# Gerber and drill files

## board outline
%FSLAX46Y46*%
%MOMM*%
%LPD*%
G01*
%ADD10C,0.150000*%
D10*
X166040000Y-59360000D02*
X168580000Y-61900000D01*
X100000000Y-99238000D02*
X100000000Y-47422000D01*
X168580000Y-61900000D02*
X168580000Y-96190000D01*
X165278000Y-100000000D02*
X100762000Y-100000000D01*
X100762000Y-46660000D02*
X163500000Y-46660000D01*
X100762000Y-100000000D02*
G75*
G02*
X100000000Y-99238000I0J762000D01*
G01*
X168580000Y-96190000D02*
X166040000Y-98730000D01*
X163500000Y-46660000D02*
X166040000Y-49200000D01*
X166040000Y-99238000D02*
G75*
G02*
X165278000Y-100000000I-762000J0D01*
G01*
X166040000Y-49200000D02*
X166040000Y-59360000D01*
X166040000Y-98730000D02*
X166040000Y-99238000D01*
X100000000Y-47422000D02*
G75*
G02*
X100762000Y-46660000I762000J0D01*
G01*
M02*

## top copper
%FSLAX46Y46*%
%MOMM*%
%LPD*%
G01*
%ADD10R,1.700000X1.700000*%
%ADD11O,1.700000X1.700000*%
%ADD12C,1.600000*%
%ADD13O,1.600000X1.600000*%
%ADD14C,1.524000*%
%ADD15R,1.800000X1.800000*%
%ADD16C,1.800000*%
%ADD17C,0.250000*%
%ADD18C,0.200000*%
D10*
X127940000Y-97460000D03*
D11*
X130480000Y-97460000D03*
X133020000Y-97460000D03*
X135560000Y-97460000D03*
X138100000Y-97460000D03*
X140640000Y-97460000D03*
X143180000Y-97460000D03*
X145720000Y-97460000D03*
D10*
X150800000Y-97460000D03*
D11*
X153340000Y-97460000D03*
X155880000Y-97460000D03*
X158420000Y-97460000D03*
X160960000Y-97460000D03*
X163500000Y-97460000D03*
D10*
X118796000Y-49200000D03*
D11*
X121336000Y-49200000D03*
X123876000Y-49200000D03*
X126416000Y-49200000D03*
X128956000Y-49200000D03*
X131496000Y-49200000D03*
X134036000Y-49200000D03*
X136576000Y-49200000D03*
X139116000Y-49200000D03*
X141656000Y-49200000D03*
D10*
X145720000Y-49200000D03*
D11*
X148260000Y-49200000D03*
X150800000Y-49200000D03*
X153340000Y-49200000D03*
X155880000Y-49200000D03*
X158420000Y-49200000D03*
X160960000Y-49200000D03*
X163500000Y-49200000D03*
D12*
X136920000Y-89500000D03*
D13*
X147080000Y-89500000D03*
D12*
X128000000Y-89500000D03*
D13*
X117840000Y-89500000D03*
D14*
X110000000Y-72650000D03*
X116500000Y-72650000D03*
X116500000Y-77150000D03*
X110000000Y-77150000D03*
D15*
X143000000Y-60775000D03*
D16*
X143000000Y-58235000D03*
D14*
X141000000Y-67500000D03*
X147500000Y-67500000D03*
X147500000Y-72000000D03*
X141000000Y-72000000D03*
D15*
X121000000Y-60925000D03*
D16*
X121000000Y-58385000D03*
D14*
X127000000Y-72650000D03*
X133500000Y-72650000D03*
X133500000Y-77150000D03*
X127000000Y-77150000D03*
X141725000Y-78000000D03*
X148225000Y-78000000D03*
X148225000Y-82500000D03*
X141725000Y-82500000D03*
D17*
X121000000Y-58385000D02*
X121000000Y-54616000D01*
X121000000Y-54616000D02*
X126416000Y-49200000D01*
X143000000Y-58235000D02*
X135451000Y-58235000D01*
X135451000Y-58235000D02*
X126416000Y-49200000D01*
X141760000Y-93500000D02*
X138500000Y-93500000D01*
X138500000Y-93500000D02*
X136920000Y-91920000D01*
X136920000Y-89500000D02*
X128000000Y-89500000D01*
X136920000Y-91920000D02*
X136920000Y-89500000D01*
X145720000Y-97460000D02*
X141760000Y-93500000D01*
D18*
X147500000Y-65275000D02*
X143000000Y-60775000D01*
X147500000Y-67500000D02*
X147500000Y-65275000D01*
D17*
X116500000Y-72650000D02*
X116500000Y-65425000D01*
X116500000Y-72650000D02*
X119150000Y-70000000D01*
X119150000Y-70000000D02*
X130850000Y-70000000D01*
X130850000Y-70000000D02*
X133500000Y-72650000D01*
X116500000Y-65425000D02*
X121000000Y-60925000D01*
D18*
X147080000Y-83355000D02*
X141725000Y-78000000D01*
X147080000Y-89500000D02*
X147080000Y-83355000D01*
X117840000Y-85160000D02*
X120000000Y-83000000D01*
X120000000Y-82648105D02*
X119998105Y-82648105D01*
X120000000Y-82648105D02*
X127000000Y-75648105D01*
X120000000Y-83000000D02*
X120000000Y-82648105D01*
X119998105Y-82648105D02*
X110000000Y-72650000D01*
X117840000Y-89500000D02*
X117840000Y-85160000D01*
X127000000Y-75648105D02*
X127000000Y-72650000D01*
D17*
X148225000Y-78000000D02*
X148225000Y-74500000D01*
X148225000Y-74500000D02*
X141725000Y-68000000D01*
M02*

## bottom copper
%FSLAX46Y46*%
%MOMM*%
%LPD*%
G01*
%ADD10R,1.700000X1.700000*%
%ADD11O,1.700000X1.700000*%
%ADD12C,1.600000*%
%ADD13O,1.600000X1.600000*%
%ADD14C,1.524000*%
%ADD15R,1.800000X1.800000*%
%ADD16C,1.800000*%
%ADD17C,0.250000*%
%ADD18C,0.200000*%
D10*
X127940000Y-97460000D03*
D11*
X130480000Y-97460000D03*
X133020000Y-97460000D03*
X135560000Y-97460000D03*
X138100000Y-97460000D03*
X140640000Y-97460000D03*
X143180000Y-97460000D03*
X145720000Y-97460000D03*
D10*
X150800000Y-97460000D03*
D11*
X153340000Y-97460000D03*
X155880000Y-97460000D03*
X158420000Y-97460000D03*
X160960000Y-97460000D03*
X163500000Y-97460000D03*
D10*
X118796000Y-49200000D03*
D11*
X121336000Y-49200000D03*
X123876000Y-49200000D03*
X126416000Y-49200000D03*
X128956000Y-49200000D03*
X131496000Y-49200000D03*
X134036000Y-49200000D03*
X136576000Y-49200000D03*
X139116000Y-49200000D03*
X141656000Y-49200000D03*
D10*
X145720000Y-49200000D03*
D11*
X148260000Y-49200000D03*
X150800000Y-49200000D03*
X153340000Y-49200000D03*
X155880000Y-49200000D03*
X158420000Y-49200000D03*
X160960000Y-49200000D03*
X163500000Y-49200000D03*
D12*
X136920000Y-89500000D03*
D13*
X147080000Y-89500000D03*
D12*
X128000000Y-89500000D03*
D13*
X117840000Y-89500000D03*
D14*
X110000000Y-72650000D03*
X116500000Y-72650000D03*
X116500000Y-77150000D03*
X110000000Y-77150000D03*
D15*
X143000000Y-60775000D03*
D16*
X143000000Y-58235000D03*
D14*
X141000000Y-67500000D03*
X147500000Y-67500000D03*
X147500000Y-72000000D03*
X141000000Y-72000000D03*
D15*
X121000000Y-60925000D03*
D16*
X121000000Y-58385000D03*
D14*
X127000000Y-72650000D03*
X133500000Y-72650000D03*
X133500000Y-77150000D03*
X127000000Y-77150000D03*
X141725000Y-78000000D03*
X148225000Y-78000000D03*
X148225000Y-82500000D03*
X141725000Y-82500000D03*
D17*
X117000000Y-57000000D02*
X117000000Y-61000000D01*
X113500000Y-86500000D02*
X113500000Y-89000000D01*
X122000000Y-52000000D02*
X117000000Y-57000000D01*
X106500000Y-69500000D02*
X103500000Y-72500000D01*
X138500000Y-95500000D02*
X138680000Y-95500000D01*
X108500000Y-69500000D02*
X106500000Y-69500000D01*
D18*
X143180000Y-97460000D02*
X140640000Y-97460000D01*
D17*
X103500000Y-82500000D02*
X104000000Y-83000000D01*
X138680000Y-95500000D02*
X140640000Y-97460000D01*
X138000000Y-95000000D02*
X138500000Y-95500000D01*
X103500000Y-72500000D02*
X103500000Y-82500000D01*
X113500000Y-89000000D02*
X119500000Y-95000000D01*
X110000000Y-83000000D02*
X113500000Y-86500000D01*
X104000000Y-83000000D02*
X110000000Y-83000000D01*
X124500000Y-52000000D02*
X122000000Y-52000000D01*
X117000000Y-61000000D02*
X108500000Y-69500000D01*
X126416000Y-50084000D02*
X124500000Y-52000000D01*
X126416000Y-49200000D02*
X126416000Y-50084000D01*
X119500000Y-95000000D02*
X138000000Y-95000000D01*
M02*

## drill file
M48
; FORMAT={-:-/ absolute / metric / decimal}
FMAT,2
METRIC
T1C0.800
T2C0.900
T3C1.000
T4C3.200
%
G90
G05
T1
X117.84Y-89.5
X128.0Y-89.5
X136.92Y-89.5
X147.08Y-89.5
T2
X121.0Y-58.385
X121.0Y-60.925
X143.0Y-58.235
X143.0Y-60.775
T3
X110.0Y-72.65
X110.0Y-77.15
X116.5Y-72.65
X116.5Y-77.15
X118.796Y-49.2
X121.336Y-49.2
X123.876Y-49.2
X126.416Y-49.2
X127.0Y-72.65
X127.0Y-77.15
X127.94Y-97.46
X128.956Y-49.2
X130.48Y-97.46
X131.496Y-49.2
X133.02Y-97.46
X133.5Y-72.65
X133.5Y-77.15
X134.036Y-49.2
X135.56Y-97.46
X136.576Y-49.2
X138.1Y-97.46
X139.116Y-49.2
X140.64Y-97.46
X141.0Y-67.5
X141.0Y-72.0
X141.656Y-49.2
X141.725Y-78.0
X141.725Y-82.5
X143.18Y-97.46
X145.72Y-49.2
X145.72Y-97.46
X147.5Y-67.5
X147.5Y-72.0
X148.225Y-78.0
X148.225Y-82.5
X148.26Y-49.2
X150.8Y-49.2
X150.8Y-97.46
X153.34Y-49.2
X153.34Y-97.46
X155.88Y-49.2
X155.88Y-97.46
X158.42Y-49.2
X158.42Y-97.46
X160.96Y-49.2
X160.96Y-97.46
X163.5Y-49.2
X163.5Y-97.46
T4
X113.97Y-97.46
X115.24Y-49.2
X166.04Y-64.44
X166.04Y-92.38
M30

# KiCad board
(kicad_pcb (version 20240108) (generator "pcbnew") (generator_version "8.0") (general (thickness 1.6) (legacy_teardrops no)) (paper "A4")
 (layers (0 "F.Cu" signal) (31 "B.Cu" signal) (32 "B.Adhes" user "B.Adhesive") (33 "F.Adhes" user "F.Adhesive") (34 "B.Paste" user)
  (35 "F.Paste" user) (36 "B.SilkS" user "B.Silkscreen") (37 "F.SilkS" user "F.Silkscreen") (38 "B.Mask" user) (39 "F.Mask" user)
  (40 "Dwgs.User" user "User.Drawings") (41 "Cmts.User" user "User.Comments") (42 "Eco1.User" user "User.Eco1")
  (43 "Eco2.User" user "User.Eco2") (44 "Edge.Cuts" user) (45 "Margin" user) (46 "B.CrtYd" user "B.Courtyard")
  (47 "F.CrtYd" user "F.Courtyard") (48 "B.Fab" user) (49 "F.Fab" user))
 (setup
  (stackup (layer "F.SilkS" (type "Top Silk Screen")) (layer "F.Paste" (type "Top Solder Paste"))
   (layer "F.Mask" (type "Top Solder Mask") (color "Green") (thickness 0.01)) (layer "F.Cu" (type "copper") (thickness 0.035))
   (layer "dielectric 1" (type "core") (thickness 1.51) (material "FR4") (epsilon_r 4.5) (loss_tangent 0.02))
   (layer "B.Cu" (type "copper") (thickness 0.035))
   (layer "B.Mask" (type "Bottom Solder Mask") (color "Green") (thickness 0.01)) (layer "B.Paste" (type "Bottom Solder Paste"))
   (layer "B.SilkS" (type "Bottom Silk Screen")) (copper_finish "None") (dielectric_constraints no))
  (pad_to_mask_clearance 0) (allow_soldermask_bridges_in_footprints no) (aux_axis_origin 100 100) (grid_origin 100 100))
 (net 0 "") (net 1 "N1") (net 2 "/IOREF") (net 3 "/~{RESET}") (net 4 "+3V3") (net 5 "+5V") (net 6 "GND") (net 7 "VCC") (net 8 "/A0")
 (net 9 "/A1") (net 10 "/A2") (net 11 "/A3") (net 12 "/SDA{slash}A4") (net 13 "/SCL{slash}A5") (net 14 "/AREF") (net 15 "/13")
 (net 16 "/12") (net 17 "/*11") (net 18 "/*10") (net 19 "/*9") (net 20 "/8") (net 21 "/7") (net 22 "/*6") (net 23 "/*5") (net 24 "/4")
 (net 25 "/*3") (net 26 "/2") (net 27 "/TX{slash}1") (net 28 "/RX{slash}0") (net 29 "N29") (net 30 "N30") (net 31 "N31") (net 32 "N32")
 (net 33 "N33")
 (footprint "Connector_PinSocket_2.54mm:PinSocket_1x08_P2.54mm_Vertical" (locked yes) (layer "F.Cu") (at 127.94 97.46 90)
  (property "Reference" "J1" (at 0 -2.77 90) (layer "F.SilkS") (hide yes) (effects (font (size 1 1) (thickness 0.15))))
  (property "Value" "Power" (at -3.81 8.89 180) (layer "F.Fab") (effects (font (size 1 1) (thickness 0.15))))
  (pad "1" thru_hole rect (at 0 0 90) (size 1.7 1.7) (drill 1) (layers "*.Cu" "*.Mask") (remove_unused_layers no) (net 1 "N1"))
  (pad "2" thru_hole oval (at 0 2.54 90) (size 1.7 1.7) (drill 1) (layers "*.Cu" "*.Mask") (remove_unused_layers no) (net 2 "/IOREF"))
  (pad "3" thru_hole oval (at 0 5.08 90) (size 1.7 1.7) (drill 1) (layers "*.Cu" "*.Mask") (remove_unused_layers no) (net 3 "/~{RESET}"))
  (pad "4" thru_hole oval (at 0 7.62 90) (size 1.7 1.7) (drill 1) (layers "*.Cu" "*.Mask") (remove_unused_layers no) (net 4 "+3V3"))
  (pad "5" thru_hole oval (at 0 10.16 90) (size 1.7 1.7) (drill 1) (layers "*.Cu" "*.Mask") (remove_unused_layers no) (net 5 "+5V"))
  (pad "6" thru_hole oval (at 0 12.7 90) (size 1.7 1.7) (drill 1) (layers "*.Cu" "*.Mask") (remove_unused_layers no) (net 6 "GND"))
  (pad "7" thru_hole oval (at 0 15.24 90) (size 1.7 1.7) (drill 1) (layers "*.Cu" "*.Mask") (remove_unused_layers no) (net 6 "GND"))
  (pad "8" thru_hole oval (at 0 17.78 90) (size 1.7 1.7) (drill 1) (layers "*.Cu" "*.Mask") (remove_unused_layers no) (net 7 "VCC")))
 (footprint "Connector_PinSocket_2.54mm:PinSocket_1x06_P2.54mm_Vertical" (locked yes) (layer "F.Cu") (at 150.8 97.46 90)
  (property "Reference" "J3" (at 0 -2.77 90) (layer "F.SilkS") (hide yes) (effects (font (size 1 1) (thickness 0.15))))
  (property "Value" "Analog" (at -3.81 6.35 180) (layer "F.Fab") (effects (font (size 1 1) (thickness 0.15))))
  (pad "1" thru_hole rect (at 0 0 90) (size 1.7 1.7) (drill 1) (layers "*.Cu" "*.Mask") (remove_unused_layers no) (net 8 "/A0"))
  (pad "2" thru_hole oval (at 0 2.54 90) (size 1.7 1.7) (drill 1) (layers "*.Cu" "*.Mask") (remove_unused_layers no) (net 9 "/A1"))
  (pad "3" thru_hole oval (at 0 5.08 90) (size 1.7 1.7) (drill 1) (layers "*.Cu" "*.Mask") (remove_unused_layers no) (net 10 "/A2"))
  (pad "4" thru_hole oval (at 0 7.62 90) (size 1.7 1.7) (drill 1) (layers "*.Cu" "*.Mask") (remove_unused_layers no) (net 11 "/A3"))
  (pad "5" thru_hole oval (at 0 10.16 90) (size 1.7 1.7) (drill 1) (layers "*.Cu" "*.Mask") (remove_unused_layers no)
   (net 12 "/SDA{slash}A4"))
  (pad "6" thru_hole oval (at 0 12.7 90) (size 1.7 1.7) (drill 1) (layers "*.Cu" "*.Mask") (remove_unused_layers no)
   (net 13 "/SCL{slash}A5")))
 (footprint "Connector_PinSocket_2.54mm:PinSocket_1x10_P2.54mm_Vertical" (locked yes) (layer "F.Cu") (at 118.796 49.2 90)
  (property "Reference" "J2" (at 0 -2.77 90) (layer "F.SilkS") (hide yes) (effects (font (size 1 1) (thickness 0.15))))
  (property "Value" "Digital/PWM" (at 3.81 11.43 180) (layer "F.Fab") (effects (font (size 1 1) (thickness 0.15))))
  (pad "1" thru_hole rect (at 0 0 90) (size 1.7 1.7) (drill 1) (layers "*.Cu" "*.Mask") (remove_unused_layers no) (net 13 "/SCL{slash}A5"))
  (pad "2" thru_hole oval (at 0 2.54 90) (size 1.7 1.7) (drill 1) (layers "*.Cu" "*.Mask") (remove_unused_layers no)
   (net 12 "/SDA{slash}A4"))
  (pad "3" thru_hole oval (at 0 5.08 90) (size 1.7 1.7) (drill 1) (layers "*.Cu" "*.Mask") (remove_unused_layers no) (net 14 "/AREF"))
  (pad "4" thru_hole oval (at 0 7.62 90) (size 1.7 1.7) (drill 1) (layers "*.Cu" "*.Mask") (remove_unused_layers no) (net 6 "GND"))
  (pad "5" thru_hole oval (at 0 10.16 90) (size 1.7 1.7) (drill 1) (layers "*.Cu" "*.Mask") (remove_unused_layers no) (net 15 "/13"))
  (pad "6" thru_hole oval (at 0 12.7 90) (size 1.7 1.7) (drill 1) (layers "*.Cu" "*.Mask") (remove_unused_layers no) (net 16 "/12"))
  (pad "7" thru_hole oval (at 0 15.24 90) (size 1.7 1.7) (drill 1) (layers "*.Cu" "*.Mask") (remove_unused_layers no) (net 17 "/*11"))
  (pad "8" thru_hole oval (at 0 17.78 90) (size 1.7 1.7) (drill 1) (layers "*.Cu" "*.Mask") (remove_unused_layers no) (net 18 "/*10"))
  (pad "9" thru_hole oval (at 0 20.32 90) (size 1.7 1.7) (drill 1) (layers "*.Cu" "*.Mask") (remove_unused_layers no) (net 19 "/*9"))
  (pad "10" thru_hole oval (at 0 22.86 90) (size 1.7 1.7) (drill 1) (layers "*.Cu" "*.Mask") (remove_unused_layers no) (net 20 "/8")))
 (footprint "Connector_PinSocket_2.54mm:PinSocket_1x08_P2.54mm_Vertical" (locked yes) (layer "F.Cu") (at 145.72 49.2 90)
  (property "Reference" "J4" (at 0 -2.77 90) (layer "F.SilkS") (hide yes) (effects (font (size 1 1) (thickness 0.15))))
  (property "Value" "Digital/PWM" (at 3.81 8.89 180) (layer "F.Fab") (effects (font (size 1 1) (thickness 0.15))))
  (pad "1" thru_hole rect (at 0 0 90) (size 1.7 1.7) (drill 1) (layers "*.Cu" "*.Mask") (remove_unused_layers no) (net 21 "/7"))
  (pad "2" thru_hole oval (at 0 2.54 90) (size 1.7 1.7) (drill 1) (layers "*.Cu" "*.Mask") (remove_unused_layers no) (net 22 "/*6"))
  (pad "3" thru_hole oval (at 0 5.08 90) (size 1.7 1.7) (drill 1) (layers "*.Cu" "*.Mask") (remove_unused_layers no) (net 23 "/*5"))
  (pad "4" thru_hole oval (at 0 7.62 90) (size 1.7 1.7) (drill 1) (layers "*.Cu" "*.Mask") (remove_unused_layers no) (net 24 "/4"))
  (pad "5" thru_hole oval (at 0 10.16 90) (size 1.7 1.7) (drill 1) (layers "*.Cu" "*.Mask") (remove_unused_layers no) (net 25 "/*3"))
  (pad "6" thru_hole oval (at 0 12.7 90) (size 1.7 1.7) (drill 1) (layers "*.Cu" "*.Mask") (remove_unused_layers no) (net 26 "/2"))
  (pad "7" thru_hole oval (at 0 15.24 90) (size 1.7 1.7) (drill 1) (layers "*.Cu" "*.Mask") (remove_unused_layers no) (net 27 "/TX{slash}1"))
  (pad "8" thru_hole oval (at 0 17.78 90) (size 1.7 1.7) (drill 1) (layers "*.Cu" "*.Mask") (remove_unused_layers no) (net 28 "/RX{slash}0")))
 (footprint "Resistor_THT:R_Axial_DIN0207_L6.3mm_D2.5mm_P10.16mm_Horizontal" (layer "F.Cu") (at 136.92 89.5)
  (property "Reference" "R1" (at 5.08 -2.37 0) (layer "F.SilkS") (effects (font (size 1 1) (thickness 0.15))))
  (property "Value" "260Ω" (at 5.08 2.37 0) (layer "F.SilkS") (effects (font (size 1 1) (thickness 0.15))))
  (pad "1" thru_hole circle (at 0 0) (size 1.6 1.6) (drill 0.8) (layers "*.Cu" "*.Mask") (remove_unused_layers no) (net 7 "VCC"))
  (pad "2" thru_hole oval (at 10.16 0) (size 1.6 1.6) (drill 0.8) (layers "*.Cu" "*.Mask") (remove_unused_layers no) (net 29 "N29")))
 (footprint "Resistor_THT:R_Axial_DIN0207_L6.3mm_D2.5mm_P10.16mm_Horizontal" (layer "F.Cu") (at 128 89.5 180)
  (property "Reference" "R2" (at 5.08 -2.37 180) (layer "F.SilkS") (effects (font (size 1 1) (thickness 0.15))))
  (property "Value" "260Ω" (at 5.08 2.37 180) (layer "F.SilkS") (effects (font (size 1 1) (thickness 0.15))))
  (pad "1" thru_hole circle (at 0 0 180) (size 1.6 1.6) (drill 0.8) (layers "*.Cu" "*.Mask") (remove_unused_layers no) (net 7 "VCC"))
  (pad "2" thru_hole oval (at 10.16 0 180) (size 1.6 1.6) (drill 0.8) (layers "*.Cu" "*.Mask") (remove_unused_layers no) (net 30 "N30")))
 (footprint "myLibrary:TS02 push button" (layer "F.Cu") (at 110 72.65)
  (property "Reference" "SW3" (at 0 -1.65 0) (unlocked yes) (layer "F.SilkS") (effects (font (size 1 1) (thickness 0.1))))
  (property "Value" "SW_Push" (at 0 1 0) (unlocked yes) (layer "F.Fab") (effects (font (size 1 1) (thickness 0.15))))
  (pad "1" thru_hole circle (at 0 0) (size 1.524 1.524) (drill 1) (layers "*.Cu" "*.Mask") (remove_unused_layers no) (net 30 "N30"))
  (pad "2" thru_hole circle (at 6.5 0) (size 1.524 1.524) (drill 1) (layers "*.Cu" "*.Mask") (remove_unused_layers no) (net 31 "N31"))
  (pad "3" thru_hole circle (at 6.5 4.5) (size 1.524 1.524) (drill 1) (layers "*.Cu" "*.Mask") (remove_unused_layers no))
  (pad "4" thru_hole circle (at 0 4.5) (size 1.524 1.524) (drill 1) (layers "*.Cu" "*.Mask") (remove_unused_layers no)))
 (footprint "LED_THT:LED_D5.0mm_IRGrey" (layer "F.Cu") (at 143 60.775 90)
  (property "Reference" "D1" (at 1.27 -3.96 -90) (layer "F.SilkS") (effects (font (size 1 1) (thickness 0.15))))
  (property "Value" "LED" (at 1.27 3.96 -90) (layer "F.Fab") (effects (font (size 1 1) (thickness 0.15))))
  (pad "1" thru_hole rect (at 0 0 90) (size 1.8 1.8) (drill 0.9) (layers "*.Cu" "*.Mask") (remove_unused_layers no) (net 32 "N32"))
  (pad "2" thru_hole circle (at 2.54 0 90) (size 1.8 1.8) (drill 0.9) (layers "*.Cu" "*.Mask") (remove_unused_layers no) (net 6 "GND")))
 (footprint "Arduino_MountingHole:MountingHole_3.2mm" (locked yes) (layer "F.Cu") (at 115.24 49.2)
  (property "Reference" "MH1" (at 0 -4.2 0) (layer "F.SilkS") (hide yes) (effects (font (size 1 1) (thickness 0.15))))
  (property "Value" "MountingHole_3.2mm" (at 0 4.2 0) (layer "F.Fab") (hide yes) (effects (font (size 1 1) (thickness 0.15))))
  (pad "" np_thru_hole circle (at 0 0) (size 3.2 3.2) (drill 3.2) (layers "*.Cu" "*.Mask")))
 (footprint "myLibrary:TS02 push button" (layer "F.Cu") (at 141 67.5)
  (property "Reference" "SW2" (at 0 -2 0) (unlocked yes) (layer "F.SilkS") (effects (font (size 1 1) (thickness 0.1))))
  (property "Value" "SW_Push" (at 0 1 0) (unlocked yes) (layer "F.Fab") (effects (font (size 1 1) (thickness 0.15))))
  (pad "1" thru_hole circle (at 0 0) (size 1.524 1.524) (drill 1) (layers "*.Cu" "*.Mask") (remove_unused_layers no) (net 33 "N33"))
  (pad "2" thru_hole circle (at 6.5 0) (size 1.524 1.524) (drill 1) (layers "*.Cu" "*.Mask") (remove_unused_layers no) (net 32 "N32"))
  (pad "3" thru_hole circle (at 6.5 4.5) (size 1.524 1.524) (drill 1) (layers "*.Cu" "*.Mask") (remove_unused_layers no))
  (pad "4" thru_hole circle (at 0 4.5) (size 1.524 1.524) (drill 1) (layers "*.Cu" "*.Mask") (remove_unused_layers no)))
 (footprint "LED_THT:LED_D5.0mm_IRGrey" (layer "F.Cu") (at 121 60.925 90)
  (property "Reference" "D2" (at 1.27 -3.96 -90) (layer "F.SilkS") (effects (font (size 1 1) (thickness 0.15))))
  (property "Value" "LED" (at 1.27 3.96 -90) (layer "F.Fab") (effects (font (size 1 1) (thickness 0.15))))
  (pad "1" thru_hole rect (at 0 0 90) (size 1.8 1.8) (drill 0.9) (layers "*.Cu" "*.Mask") (remove_unused_layers no) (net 31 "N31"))
  (pad "2" thru_hole circle (at 2.54 0 90) (size 1.8 1.8) (drill 0.9) (layers "*.Cu" "*.Mask") (remove_unused_layers no) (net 6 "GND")))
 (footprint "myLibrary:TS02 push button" (layer "F.Cu") (at 127 72.65)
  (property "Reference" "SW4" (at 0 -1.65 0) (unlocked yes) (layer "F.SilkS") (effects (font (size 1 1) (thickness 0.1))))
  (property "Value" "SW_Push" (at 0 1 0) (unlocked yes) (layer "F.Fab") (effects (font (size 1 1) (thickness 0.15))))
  (pad "1" thru_hole circle (at 0 0) (size 1.524 1.524) (drill 1) (layers "*.Cu" "*.Mask") (remove_unused_layers no) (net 30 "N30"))
  (pad "2" thru_hole circle (at 6.5 0) (size 1.524 1.524) (drill 1) (layers "*.Cu" "*.Mask") (remove_unused_layers no) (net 31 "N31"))
  (pad "3" thru_hole circle (at 6.5 4.5) (size 1.524 1.524) (drill 1) (layers "*.Cu" "*.Mask") (remove_unused_layers no))
  (pad "4" thru_hole circle (at 0 4.5) (size 1.524 1.524) (drill 1) (layers "*.Cu" "*.Mask") (remove_unused_layers no)))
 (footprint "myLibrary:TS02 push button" (layer "F.Cu") (at 141.725 78)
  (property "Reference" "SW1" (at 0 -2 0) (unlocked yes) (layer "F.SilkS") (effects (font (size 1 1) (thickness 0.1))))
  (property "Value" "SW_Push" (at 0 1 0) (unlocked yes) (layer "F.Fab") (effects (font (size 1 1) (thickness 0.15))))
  (pad "1" thru_hole circle (at 0 0) (size 1.524 1.524) (drill 1) (layers "*.Cu" "*.Mask") (remove_unused_layers no) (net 29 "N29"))
  (pad "2" thru_hole circle (at 6.5 0) (size 1.524 1.524) (drill 1) (layers "*.Cu" "*.Mask") (remove_unused_layers no) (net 33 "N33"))
  (pad "3" thru_hole circle (at 6.5 4.5) (size 1.524 1.524) (drill 1) (layers "*.Cu" "*.Mask") (remove_unused_layers no))
  (pad "4" thru_hole circle (at 0 4.5) (size 1.524 1.524) (drill 1) (layers "*.Cu" "*.Mask") (remove_unused_layers no)))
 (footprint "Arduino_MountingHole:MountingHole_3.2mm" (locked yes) (layer "F.Cu") (at 113.97 97.46)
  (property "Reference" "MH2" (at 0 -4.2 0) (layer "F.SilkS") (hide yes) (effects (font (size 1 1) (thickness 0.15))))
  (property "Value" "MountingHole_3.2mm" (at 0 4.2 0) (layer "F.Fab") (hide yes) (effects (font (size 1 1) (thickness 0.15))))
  (pad "" np_thru_hole circle (at 0 0) (size 3.2 3.2) (drill 3.2) (layers "*.Cu" "*.Mask")))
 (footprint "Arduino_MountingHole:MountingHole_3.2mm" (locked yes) (layer "F.Cu") (at 166.04 64.44)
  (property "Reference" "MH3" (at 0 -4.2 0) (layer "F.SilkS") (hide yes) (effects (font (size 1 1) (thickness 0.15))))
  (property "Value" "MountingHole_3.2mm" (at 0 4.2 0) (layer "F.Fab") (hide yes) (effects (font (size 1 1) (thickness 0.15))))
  (pad "" np_thru_hole circle (at 0 0) (size 3.2 3.2) (drill 3.2) (layers "*.Cu" "*.Mask")))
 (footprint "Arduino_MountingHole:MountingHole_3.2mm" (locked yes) (layer "F.Cu") (at 166.04 92.38)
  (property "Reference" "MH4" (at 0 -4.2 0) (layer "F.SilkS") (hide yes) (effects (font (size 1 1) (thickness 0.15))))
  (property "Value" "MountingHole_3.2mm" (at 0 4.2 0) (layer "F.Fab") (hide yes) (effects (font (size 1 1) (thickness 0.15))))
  (pad "" np_thru_hole circle (at 0 0) (size 3.2 3.2) (drill 3.2) (layers "*.Cu" "*.Mask")))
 (gr_line (start 166.04 59.36) (end 168.58 61.9) (stroke (width 0.15) (type solid)) (layer "Edge.Cuts"))
 (gr_line (start 100 99.238) (end 100 47.422) (stroke (width 0.15) (type solid)) (layer "Edge.Cuts"))
 (gr_line (start 168.58 61.9) (end 168.58 96.19) (stroke (width 0.15) (type solid)) (layer "Edge.Cuts"))
 (gr_line (start 165.278 100) (end 100.762 100) (stroke (width 0.15) (type solid)) (layer "Edge.Cuts"))
 (gr_line (start 100.762 46.66) (end 163.5 46.66) (stroke (width 0.15) (type solid)) (layer "Edge.Cuts"))
 (gr_arc (start 100.762 100) (mid 100.223185 99.776815) (end 100 99.238) (stroke (width 0.15) (type solid)) (layer "Edge.Cuts"))
 (gr_line (start 168.58 96.19) (end 166.04 98.73) (stroke (width 0.15) (type solid)) (layer "Edge.Cuts"))
 (gr_line (start 163.5 46.66) (end 166.04 49.2) (stroke (width 0.15) (type solid)) (layer "Edge.Cuts"))
 (gr_arc (start 166.04 99.238) (mid 165.816815 99.776815) (end 165.278 100) (stroke (width 0.15) (type solid)) (layer "Edge.Cuts"))
 (gr_line (start 166.04 49.2) (end 166.04 59.36) (stroke (width 0.15) (type solid)) (layer "Edge.Cuts"))
 (gr_line (start 166.04 98.73) (end 166.04 99.238) (stroke (width 0.15) (type solid)) (layer "Edge.Cuts"))
 (gr_arc (start 100 47.422) (mid 100.223185 46.883185) (end 100.762 46.66) (stroke (width 0.15) (type solid)) (layer "Edge.Cuts"))
 (segment (start 121 58.385) (end 121 54.616) (width 0.25) (layer "F.Cu") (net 6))
 (segment (start 121 54.616) (end 126.416 49.2) (width 0.25) (layer "F.Cu") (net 6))
 (segment (start 143 58.235) (end 135.451 58.235) (width 0.25) (layer "F.Cu") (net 6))
 (segment (start 135.451 58.235) (end 126.416 49.2) (width 0.25) (layer "F.Cu") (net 6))
 (segment (start 117 57) (end 117 61) (width 0.25) (layer "B.Cu") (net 6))
 (segment (start 113.5 86.5) (end 113.5 89) (width 0.25) (layer "B.Cu") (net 6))
 (segment (start 122 52) (end 117 57) (width 0.25) (layer "B.Cu") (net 6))
 (segment (start 106.5 69.5) (end 103.5 72.5) (width 0.25) (layer "B.Cu") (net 6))
 (segment (start 138.5 95.5) (end 138.68 95.5) (width 0.25) (layer "B.Cu") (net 6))
 (segment (start 108.5 69.5) (end 106.5 69.5) (width 0.25) (layer "B.Cu") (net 6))
 (segment (start 143.18 97.46) (end 140.64 97.46) (width 0.2) (layer "B.Cu") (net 6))
 (segment (start 103.5 82.5) (end 104 83) (width 0.25) (layer "B.Cu") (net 6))
 (segment (start 138.68 95.5) (end 140.64 97.46) (width 0.25) (layer "B.Cu") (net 6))
 (segment (start 138 95) (end 138.5 95.5) (width 0.25) (layer "B.Cu") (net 6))
 (segment (start 103.5 72.5) (end 103.5 82.5) (width 0.25) (layer "B.Cu") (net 6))
 (segment (start 113.5 89) (end 119.5 95) (width 0.25) (layer "B.Cu") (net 6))
 (segment (start 110 83) (end 113.5 86.5) (width 0.25) (layer "B.Cu") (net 6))
 (segment (start 104 83) (end 110 83) (width 0.25) (layer "B.Cu") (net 6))
 (segment (start 124.5 52) (end 122 52) (width 0.25) (layer "B.Cu") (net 6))
 (segment (start 117 61) (end 108.5 69.5) (width 0.25) (layer "B.Cu") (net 6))
 (segment (start 126.416 50.084) (end 124.5 52) (width 0.25) (layer "B.Cu") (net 6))
 (segment (start 126.416 49.2) (end 126.416 50.084) (width 0.25) (layer "B.Cu") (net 6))
 (segment (start 119.5 95) (end 138 95) (width 0.25) (layer "B.Cu") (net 6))
 (segment (start 141.76 93.5) (end 138.5 93.5) (width 0.25) (layer "F.Cu") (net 7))
 (segment (start 138.5 93.5) (end 136.92 91.92) (width 0.25) (layer "F.Cu") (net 7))
 (segment (start 136.92 89.5) (end 128 89.5) (width 0.25) (layer "F.Cu") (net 7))
 (segment (start 136.92 91.92) (end 136.92 89.5) (width 0.25) (layer "F.Cu") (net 7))
 (segment (start 145.72 97.46) (end 141.76 93.5) (width 0.25) (layer "F.Cu") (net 7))
 (segment (start 147.5 65.275) (end 143 60.775) (width 0.2) (layer "F.Cu") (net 32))
 (segment (start 147.5 67.5) (end 147.5 65.275) (width 0.2) (layer "F.Cu") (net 32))
 (segment (start 116.5 72.65) (end 116.5 65.425) (width 0.25) (layer "F.Cu") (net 31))
 (segment (start 116.5 72.65) (end 119.15 70) (width 0.25) (layer "F.Cu") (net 31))
 (segment (start 119.15 70) (end 130.85 70) (width 0.25) (layer "F.Cu") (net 31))
 (segment (start 130.85 70) (end 133.5 72.65) (width 0.25) (layer "F.Cu") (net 31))
 (segment (start 116.5 65.425) (end 121 60.925) (width 0.25) (layer "F.Cu") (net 31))
 (segment (start 147.08 83.355) (end 141.725 78) (width 0.2) (layer "F.Cu") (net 29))
 (segment (start 147.08 89.5) (end 147.08 83.355) (width 0.2) (layer "F.Cu") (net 29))
 (segment (start 117.84 85.16) (end 120 83) (width 0.2) (layer "F.Cu") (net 30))
 (segment (start 120 82.648105) (end 119.998105 82.648105) (width 0.2) (layer "F.Cu") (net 30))
 (segment (start 120 82.648105) (end 127 75.648105) (width 0.2) (layer "F.Cu") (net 30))
 (segment (start 120 83) (end 120 82.648105) (width 0.2) (layer "F.Cu") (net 30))
 (segment (start 119.998105 82.648105) (end 110 72.65) (width 0.2) (layer "F.Cu") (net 30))
 (segment (start 117.84 89.5) (end 117.84 85.16) (width 0.2) (layer "F.Cu") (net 30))
 (segment (start 127 75.648105) (end 127 72.65) (width 0.2) (layer "F.Cu") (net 30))
 (segment (start 148.225 78) (end 148.225 74.5) (width 0.25) (layer "F.Cu") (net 33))
 (segment (start 148.225 74.5) (end 141.725 68) (width 0.25) (layer "F.Cu") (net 33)))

